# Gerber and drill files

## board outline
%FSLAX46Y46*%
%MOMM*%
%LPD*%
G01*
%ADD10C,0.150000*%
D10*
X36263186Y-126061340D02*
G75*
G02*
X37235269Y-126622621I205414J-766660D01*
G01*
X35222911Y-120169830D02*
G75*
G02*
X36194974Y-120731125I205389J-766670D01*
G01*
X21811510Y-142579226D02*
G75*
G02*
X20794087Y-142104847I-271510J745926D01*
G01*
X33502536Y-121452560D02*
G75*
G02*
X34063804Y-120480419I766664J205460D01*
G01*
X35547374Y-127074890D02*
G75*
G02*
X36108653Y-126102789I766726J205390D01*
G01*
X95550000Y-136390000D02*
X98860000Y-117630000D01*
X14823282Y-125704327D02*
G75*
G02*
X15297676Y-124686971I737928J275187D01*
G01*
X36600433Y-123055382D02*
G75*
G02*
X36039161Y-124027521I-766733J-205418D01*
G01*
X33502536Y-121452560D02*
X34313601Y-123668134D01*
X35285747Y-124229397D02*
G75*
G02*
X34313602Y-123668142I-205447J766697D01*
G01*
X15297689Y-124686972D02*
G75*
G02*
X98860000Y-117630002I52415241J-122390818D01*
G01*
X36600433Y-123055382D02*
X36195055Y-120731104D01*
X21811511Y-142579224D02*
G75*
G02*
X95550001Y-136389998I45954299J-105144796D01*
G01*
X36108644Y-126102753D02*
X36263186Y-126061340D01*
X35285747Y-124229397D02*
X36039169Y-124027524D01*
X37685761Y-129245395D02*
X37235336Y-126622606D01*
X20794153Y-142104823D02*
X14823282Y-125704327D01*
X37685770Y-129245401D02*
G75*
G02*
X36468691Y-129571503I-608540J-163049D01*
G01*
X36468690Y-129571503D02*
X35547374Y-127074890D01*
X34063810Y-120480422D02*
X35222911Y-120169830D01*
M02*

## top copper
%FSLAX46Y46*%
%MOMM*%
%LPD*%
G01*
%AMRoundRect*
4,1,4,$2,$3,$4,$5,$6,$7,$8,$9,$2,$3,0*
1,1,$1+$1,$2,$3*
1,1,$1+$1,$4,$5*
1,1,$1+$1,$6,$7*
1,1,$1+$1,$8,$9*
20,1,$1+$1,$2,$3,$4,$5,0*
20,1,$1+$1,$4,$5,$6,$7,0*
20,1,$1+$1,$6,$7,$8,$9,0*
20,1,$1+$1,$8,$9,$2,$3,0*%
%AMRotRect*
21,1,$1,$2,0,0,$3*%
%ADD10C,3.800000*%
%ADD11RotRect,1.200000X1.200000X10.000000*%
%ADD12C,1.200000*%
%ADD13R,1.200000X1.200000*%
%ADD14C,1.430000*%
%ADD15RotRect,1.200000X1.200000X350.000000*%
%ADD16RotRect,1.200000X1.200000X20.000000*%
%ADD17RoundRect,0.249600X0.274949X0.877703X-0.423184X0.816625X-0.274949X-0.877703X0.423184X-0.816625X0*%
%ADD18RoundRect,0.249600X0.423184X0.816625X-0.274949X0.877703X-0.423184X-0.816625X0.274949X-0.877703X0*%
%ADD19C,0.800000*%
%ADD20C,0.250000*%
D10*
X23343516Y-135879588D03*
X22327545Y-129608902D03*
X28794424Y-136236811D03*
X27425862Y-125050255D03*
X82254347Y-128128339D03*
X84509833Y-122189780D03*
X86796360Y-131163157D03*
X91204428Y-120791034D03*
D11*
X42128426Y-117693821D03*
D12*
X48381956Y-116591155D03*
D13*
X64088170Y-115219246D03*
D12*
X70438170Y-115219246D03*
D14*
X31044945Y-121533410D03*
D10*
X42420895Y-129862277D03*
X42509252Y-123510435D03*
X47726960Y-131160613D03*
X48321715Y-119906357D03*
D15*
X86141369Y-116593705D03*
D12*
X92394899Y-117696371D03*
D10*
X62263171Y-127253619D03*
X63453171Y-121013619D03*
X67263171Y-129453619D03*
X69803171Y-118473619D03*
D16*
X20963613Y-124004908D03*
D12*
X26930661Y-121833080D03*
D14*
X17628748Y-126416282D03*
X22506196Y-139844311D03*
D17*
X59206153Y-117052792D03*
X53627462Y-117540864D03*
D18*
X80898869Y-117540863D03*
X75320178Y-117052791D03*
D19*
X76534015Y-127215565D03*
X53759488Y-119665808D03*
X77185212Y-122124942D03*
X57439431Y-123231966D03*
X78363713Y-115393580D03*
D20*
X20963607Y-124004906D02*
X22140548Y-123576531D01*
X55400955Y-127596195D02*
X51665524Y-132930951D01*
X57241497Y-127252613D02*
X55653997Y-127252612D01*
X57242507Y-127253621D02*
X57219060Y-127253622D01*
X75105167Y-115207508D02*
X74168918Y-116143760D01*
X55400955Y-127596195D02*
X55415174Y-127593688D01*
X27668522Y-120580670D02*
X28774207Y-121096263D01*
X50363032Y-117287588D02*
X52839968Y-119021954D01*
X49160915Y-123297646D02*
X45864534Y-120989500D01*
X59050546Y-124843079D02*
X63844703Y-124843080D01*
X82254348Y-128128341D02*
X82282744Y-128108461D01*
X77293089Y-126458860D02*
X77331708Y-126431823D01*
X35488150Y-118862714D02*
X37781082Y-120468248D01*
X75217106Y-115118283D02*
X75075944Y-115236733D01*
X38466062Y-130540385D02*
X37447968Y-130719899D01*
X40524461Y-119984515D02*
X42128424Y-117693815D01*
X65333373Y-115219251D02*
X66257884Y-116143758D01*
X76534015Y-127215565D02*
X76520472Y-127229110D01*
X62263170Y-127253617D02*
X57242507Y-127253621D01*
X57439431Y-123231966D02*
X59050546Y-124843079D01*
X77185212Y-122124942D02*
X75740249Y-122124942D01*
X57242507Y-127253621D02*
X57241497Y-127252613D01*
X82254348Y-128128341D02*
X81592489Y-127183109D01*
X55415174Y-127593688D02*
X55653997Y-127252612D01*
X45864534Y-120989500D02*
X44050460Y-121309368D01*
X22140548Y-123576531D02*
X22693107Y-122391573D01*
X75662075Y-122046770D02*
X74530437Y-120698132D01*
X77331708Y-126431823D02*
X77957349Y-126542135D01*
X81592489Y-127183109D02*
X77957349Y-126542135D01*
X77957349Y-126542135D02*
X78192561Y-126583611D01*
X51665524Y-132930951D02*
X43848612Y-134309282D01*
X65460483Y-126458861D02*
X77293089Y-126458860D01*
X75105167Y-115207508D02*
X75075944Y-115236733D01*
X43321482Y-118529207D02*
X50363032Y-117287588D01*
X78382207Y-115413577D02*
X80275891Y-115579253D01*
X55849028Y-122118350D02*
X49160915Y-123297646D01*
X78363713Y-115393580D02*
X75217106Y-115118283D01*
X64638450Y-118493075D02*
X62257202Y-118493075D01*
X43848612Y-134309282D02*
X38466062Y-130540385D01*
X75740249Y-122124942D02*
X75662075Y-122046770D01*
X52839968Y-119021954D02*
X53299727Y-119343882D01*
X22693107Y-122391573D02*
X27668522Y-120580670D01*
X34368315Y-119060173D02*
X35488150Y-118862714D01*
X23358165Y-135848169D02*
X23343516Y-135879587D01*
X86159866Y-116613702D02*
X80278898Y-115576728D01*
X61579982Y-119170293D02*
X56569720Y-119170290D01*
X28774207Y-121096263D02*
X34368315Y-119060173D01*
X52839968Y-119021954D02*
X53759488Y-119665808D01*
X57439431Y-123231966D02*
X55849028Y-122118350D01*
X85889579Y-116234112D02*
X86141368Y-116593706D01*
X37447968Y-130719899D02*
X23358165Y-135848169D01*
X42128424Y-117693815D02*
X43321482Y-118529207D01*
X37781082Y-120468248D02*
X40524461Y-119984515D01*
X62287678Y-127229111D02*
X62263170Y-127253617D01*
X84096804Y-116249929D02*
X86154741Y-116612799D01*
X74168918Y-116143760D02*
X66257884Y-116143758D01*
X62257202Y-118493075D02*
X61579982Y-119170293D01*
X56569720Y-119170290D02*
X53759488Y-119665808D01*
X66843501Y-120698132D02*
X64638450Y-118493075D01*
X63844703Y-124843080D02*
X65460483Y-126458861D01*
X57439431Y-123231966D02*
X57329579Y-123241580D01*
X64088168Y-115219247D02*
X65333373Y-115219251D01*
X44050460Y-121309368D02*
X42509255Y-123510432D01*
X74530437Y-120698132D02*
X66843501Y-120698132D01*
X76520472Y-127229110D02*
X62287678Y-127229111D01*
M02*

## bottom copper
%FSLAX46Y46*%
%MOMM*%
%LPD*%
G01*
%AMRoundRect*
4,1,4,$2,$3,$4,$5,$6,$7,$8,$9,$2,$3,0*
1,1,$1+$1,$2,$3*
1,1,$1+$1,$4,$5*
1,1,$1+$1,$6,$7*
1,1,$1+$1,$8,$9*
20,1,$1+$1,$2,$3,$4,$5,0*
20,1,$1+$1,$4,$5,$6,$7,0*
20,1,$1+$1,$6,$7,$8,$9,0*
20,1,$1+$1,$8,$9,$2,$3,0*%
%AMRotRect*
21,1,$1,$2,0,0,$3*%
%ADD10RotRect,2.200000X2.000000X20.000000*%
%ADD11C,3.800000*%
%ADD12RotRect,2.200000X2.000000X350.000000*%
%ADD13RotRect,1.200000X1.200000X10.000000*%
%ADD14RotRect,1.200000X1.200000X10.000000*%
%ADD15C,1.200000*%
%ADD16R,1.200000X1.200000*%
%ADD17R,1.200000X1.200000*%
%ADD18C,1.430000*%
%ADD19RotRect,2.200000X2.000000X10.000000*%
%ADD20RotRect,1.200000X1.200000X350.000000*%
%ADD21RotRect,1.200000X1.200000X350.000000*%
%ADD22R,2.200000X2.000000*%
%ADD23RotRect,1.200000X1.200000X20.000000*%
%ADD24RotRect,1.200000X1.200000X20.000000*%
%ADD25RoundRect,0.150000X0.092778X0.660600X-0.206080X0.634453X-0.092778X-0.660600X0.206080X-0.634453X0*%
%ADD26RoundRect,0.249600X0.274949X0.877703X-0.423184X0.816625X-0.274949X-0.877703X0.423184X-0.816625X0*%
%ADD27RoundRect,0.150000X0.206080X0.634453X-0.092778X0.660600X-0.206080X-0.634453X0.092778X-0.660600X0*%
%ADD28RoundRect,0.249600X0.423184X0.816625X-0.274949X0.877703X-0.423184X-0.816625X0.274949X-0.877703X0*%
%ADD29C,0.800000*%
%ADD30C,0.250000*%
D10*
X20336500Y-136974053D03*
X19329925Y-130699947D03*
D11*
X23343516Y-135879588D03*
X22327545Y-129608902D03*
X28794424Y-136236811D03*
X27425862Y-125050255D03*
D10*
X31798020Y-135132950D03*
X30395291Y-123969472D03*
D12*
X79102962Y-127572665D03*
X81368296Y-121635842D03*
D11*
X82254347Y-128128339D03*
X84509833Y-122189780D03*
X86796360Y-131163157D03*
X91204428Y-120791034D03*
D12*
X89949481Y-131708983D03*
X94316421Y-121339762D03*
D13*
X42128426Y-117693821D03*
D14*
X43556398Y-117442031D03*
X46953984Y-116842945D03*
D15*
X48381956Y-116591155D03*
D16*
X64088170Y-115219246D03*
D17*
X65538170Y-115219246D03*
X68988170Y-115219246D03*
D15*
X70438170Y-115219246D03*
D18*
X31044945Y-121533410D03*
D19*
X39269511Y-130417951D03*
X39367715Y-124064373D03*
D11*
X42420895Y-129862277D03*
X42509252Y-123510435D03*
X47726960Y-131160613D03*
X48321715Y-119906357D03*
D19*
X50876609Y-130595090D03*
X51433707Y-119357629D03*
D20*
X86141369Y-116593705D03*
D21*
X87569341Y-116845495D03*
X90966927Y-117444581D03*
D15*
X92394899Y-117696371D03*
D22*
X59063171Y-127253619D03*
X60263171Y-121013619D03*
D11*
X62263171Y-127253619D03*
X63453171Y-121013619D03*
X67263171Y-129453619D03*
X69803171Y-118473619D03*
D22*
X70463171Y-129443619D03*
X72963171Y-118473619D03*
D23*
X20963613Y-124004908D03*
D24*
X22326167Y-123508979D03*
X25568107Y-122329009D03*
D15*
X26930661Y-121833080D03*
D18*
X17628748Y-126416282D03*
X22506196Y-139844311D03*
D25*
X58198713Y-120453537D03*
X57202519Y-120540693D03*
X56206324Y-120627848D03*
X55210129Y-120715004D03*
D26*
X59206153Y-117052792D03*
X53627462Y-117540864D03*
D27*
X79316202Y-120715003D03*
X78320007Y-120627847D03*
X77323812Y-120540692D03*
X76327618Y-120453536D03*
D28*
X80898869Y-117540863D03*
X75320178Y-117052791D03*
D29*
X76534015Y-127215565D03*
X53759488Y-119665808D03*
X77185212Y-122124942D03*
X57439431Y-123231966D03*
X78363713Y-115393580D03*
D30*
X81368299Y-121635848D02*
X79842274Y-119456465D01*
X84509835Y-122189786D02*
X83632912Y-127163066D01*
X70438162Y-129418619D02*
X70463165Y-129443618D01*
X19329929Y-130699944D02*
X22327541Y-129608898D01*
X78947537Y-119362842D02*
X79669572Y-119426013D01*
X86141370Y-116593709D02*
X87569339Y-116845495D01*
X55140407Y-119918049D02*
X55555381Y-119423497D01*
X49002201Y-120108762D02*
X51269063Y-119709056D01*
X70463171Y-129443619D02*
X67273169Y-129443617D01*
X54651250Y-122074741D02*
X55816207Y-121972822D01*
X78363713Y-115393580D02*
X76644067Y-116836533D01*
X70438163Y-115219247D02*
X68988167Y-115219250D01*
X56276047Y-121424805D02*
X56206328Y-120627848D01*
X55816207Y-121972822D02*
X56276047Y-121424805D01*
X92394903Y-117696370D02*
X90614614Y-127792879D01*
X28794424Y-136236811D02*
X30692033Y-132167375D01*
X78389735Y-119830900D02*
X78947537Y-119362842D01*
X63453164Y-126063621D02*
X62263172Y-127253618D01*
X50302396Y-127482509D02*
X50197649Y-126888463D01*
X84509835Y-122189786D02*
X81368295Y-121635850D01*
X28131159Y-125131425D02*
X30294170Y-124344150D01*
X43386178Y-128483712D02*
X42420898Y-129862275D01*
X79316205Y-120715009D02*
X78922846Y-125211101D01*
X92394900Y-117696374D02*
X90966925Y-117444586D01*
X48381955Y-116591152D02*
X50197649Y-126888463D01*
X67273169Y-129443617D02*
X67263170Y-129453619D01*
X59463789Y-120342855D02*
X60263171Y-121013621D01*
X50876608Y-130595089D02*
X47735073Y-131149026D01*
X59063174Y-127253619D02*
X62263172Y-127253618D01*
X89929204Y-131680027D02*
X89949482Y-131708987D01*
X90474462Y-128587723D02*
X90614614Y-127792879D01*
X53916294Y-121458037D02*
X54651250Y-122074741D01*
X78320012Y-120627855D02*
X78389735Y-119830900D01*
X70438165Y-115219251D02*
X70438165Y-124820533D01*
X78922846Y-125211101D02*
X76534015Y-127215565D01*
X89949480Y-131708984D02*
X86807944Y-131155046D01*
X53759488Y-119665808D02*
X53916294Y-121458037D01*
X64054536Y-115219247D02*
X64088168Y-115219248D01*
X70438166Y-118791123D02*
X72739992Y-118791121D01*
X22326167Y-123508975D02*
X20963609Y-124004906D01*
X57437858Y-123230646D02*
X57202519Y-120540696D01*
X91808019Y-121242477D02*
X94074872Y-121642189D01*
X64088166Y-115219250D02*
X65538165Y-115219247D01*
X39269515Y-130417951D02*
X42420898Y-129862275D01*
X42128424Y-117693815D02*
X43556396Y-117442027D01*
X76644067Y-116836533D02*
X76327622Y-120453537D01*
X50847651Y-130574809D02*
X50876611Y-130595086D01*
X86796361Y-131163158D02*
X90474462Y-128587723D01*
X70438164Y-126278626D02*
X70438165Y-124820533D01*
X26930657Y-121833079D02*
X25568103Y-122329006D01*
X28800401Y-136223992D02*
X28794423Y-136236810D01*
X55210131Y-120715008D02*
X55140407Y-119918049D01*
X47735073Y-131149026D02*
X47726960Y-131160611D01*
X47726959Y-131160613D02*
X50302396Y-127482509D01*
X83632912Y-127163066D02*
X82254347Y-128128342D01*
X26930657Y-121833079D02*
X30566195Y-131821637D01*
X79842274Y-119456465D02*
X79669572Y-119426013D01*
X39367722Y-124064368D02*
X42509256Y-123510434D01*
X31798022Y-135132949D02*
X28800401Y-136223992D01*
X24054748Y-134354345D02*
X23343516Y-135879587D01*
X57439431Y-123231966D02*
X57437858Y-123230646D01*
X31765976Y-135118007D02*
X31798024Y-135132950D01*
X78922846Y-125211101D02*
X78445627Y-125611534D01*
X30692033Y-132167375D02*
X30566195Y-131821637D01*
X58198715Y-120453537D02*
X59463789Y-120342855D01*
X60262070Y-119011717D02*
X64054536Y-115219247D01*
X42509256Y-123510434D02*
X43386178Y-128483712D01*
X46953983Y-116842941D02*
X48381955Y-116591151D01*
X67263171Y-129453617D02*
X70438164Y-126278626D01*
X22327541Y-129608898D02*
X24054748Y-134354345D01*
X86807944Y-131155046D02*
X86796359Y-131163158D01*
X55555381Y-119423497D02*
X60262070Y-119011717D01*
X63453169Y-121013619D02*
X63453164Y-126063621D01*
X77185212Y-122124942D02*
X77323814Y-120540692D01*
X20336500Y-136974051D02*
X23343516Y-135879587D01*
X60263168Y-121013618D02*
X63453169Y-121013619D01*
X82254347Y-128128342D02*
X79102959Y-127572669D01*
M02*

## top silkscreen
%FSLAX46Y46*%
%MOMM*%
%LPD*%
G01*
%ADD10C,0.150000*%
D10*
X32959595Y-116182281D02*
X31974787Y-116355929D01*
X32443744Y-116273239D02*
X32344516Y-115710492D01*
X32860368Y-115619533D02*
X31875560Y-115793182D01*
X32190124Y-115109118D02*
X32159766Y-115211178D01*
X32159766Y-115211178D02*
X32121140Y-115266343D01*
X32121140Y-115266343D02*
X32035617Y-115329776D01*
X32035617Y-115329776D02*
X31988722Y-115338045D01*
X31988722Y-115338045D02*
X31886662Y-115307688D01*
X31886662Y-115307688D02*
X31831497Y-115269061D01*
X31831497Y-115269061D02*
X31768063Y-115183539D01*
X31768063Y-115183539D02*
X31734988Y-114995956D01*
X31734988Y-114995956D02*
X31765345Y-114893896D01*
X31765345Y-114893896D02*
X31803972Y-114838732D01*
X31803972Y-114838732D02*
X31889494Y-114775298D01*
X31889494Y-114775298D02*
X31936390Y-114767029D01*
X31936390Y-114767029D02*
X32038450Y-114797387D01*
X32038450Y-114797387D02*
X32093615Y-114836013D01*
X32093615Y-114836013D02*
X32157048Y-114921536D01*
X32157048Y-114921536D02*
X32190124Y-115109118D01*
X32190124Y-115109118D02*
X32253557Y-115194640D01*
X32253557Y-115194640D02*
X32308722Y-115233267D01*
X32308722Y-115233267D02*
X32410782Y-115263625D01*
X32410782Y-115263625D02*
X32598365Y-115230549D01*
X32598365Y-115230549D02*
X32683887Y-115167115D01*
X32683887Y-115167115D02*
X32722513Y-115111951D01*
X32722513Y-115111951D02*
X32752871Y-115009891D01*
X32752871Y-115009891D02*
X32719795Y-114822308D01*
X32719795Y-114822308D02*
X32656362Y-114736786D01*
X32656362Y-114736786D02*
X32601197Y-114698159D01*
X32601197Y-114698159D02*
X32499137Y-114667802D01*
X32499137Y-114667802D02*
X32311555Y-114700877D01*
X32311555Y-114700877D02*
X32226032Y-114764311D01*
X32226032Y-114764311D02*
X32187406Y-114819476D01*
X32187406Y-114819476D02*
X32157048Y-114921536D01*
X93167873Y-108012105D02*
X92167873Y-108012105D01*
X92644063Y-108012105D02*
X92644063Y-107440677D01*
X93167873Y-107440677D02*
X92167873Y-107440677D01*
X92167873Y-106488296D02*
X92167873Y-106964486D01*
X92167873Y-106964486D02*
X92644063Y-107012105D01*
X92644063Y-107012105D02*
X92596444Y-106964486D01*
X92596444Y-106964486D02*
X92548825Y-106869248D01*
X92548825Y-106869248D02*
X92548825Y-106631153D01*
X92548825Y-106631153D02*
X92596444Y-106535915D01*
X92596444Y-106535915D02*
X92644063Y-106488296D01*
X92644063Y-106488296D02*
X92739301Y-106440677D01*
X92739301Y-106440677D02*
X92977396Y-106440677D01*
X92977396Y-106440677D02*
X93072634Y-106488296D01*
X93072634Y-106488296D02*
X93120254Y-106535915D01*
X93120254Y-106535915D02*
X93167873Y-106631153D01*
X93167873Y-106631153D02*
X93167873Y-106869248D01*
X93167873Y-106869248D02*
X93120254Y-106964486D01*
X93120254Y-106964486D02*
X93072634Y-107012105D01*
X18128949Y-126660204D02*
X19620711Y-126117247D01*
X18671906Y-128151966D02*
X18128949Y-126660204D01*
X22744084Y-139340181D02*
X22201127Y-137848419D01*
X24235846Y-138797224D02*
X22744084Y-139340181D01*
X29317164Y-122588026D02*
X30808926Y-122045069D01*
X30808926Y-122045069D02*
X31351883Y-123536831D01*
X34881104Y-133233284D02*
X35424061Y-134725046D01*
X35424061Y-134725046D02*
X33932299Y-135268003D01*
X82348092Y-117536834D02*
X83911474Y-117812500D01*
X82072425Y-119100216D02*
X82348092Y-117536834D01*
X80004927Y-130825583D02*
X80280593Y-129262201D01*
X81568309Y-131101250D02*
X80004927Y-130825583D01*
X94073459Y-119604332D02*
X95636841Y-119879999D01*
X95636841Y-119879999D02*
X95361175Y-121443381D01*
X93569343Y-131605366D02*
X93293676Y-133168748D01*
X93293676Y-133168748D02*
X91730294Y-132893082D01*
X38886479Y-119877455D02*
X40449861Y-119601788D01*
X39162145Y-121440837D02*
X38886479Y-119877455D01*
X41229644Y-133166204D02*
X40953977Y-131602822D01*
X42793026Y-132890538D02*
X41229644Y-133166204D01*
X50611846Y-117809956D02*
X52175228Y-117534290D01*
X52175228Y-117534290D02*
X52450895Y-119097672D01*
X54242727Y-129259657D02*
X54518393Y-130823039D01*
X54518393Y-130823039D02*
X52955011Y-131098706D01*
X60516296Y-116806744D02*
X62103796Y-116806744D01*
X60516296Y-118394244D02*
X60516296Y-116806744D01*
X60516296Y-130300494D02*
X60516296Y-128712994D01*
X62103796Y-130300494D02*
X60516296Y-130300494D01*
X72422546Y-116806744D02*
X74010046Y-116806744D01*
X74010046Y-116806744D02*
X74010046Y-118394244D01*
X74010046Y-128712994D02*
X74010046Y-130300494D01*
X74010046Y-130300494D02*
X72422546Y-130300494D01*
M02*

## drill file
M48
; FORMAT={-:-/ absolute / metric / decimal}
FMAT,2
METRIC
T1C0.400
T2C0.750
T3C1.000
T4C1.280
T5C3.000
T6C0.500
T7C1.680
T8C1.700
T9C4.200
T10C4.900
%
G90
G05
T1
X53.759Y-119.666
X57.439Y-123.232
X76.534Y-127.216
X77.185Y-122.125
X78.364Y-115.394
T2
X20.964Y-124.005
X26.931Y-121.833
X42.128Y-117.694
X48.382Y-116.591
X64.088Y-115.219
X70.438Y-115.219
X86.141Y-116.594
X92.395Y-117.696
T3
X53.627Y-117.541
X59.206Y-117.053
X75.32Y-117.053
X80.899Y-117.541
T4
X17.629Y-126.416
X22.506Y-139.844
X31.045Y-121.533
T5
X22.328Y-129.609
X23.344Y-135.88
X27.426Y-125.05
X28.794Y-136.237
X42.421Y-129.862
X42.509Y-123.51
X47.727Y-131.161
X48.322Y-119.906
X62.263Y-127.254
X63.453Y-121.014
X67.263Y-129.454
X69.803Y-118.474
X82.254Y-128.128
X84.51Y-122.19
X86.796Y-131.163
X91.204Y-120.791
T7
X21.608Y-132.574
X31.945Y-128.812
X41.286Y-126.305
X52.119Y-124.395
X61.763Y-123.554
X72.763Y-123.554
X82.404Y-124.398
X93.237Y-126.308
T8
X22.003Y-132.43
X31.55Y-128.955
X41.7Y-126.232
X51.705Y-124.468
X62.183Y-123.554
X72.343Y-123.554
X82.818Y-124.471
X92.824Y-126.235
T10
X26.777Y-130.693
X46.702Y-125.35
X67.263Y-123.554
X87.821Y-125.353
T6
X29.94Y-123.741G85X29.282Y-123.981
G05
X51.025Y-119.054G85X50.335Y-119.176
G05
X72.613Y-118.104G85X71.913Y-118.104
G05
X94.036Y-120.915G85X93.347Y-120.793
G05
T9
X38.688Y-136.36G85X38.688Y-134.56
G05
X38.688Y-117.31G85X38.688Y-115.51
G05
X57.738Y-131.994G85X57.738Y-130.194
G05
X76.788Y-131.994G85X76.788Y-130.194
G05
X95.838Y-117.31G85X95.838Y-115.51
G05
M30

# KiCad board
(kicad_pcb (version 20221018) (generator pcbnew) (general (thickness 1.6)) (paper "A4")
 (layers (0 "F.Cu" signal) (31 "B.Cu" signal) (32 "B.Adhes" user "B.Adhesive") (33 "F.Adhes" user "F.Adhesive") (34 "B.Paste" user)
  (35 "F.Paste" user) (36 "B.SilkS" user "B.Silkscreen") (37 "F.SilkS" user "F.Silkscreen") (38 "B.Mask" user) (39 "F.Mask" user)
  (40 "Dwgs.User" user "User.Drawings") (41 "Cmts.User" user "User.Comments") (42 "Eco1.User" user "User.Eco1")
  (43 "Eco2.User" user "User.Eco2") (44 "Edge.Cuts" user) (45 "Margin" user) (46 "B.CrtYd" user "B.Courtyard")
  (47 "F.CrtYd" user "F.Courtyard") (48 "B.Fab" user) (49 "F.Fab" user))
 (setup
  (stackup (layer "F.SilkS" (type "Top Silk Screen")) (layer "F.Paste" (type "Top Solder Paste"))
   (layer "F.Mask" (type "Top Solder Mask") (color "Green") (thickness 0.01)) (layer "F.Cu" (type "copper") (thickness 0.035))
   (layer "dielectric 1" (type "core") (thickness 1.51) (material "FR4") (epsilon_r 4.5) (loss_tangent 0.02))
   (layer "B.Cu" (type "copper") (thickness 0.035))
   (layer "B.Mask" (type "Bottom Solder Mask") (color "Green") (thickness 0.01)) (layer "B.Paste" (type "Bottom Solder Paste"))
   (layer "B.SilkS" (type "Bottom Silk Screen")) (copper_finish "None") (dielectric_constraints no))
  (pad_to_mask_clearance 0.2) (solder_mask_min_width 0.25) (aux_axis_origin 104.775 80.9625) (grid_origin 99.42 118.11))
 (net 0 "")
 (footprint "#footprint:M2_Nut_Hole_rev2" (layer "F.Cu") (at 38.688167 135.459876 90)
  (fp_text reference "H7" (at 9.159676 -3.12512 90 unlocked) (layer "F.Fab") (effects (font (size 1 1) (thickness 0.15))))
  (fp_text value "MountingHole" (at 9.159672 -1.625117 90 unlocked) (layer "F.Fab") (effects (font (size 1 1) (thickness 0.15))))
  (pad "" np_thru_hole oval (at 0 0 90) (size 6 4.2) (drill oval 6 4.2) (layers "F&B.Cu" "*.Mask")))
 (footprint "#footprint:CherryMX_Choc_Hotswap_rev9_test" (layer "F.Cu") (at 26.776505 130.692625 20)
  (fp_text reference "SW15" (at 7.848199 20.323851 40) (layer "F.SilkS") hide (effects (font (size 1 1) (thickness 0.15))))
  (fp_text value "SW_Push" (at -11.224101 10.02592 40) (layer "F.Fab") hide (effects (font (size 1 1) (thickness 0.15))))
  (fp_line (start -6.746875 -6.746875) (end -5.159375 -6.746875) (stroke (width 0.15) (type solid)) (layer "F.SilkS"))
  (fp_line (start -6.746875 -5.159375) (end -6.746875 -6.746875) (stroke (width 0.15) (type solid)) (layer "F.SilkS"))
  (fp_line (start -6.746875 6.746875) (end -6.746875 5.159375) (stroke (width 0.15) (type solid)) (layer "F.SilkS"))
  (fp_line (start -5.159375 6.746875) (end -6.746875 6.746875) (stroke (width 0.15) (type solid)) (layer "F.SilkS"))
  (fp_line (start 5.159375 -6.746875) (end 6.746875 -6.746875) (stroke (width 0.15) (type solid)) (layer "F.SilkS"))
  (fp_line (start 6.746875 -6.746875) (end 6.746875 -5.159375) (stroke (width 0.15) (type solid)) (layer "F.SilkS"))
  (fp_line (start 6.746875 5.159375) (end 6.746875 6.746875) (stroke (width 0.15) (type solid)) (layer "F.SilkS"))
  (fp_line (start 6.746875 6.746875) (end 5.159375 6.746875) (stroke (width 0.15) (type solid)) (layer "F.SilkS"))
  (pad "" np_thru_hole circle (at -5.5 0 110) (size 1.68 1.68) (drill 1.68) (layers "F&B.Cu" "*.Mask"))
  (pad "" np_thru_hole circle (at -5.08 0 20) (size 1.7 1.7) (drill 1.7) (layers "*.Cu" "*.Mask"))
  (pad "" np_thru_hole circle (at 0 0 110) (size 4.9 4.9) (drill 4.9) (layers "F&B.Cu" "*.Mask"))
  (pad "" np_thru_hole oval (at 5 -5.45 200) (size 1.2 0.5) (drill oval 1.2 0.5) (layers "F&B.Cu" "*.Mask"))
  (pad "" np_thru_hole circle (at 5.08 0 20) (size 1.7 1.7) (drill 1.7) (layers "*.Cu" "*.Mask"))
  (pad "" np_thru_hole circle (at 5.5 0 110) (size 1.68 1.68) (drill 1.68) (layers "F&B.Cu" "*.Mask"))
  (pad "1" smd rect (at -8.2 3.7 20) (size 2.2 2) (layers "B.Cu" "B.Paste" "B.Mask"))
  (pad "1" smd rect (at -7 -2.54 20) (size 2.2 2) (layers "B.Cu" "B.Paste" "B.Mask"))
  (pad "1" thru_hole circle (at -5 3.7 110) (size 3.8 3.8) (drill 3) (layers "*.Cu" "B.Mask"))
  (pad "1" thru_hole circle (at -3.81 -2.54 200) (size 3.8 3.8) (drill 3) (layers "*.Cu" "B.Mask"))
  (pad "2" thru_hole circle (at 0 5.9 110) (size 3.8 3.8) (drill 3) (layers "*.Cu" "B.Mask"))
  (pad "2" thru_hole circle (at 2.54 -5.08 200) (size 3.8 3.8) (drill 3) (layers "*.Cu" "B.Mask"))
  (pad "2" smd rect (at 3.2 5.89 20) (size 2.2 2) (layers "B.Cu" "B.Paste" "B.Mask"))
  (pad "2" smd rect (at 5.7 -5.08 20) (size 2.2 2) (layers "B.Cu" "B.Paste" "B.Mask")))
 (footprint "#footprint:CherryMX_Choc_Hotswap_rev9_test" (layer "F.Cu") (at 87.820884 125.352791 -10)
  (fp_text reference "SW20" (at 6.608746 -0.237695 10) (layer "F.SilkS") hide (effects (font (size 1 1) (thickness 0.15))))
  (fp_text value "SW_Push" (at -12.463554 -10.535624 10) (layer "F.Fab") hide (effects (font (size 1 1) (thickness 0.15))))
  (fp_line (start -6.746875 -6.746875) (end -5.159375 -6.746875) (stroke (width 0.15) (type solid)) (layer "F.SilkS"))
  (fp_line (start -6.746875 -5.159375) (end -6.746875 -6.746875) (stroke (width 0.15) (type solid)) (layer "F.SilkS"))
  (fp_line (start -6.746875 6.746875) (end -6.746875 5.159375) (stroke (width 0.15) (type solid)) (layer "F.SilkS"))
  (fp_line (start -5.159375 6.746875) (end -6.746875 6.746875) (stroke (width 0.15) (type solid)) (layer "F.SilkS"))
  (fp_line (start 5.159375 -6.746875) (end 6.746875 -6.746875) (stroke (width 0.15) (type solid)) (layer "F.SilkS"))
  (fp_line (start 6.746875 -6.746875) (end 6.746875 -5.159375) (stroke (width 0.15) (type solid)) (layer "F.SilkS"))
  (fp_line (start 6.746875 5.159375) (end 6.746875 6.746875) (stroke (width 0.15) (type solid)) (layer "F.SilkS"))
  (fp_line (start 6.746875 6.746875) (end 5.159375 6.746875) (stroke (width 0.15) (type solid)) (layer "F.SilkS"))
  (pad "" np_thru_hole circle (at -5.5 0 80) (size 1.68 1.68) (drill 1.68) (layers "F&B.Cu" "*.Mask"))
  (pad "" np_thru_hole circle (at -5.08 0 350) (size 1.7 1.7) (drill 1.7) (layers "*.Cu" "*.Mask"))
  (pad "" np_thru_hole circle (at 0 0 80) (size 4.9 4.9) (drill 4.9) (layers "F&B.Cu" "*.Mask"))
  (pad "" np_thru_hole oval (at 5 -5.45 170) (size 1.2 0.5) (drill oval 1.2 0.5) (layers "F&B.Cu" "*.Mask"))
  (pad "" np_thru_hole circle (at 5.08 0 350) (size 1.7 1.7) (drill 1.7) (layers "*.Cu" "*.Mask"))
  (pad "" np_thru_hole circle (at 5.5 0 80) (size 1.68 1.68) (drill 1.68) (layers "F&B.Cu" "*.Mask"))
  (pad "1" smd rect (at -8.2 3.7 350) (size 2.2 2) (layers "B.Cu" "B.Paste" "B.Mask"))
  (pad "1" smd rect (at -7 -2.54 350) (size 2.2 2) (layers "B.Cu" "B.Paste" "B.Mask"))
  (pad "1" thru_hole circle (at -5 3.7 80) (size 3.8 3.8) (drill 3) (layers "*.Cu" "B.Mask"))
  (pad "1" thru_hole circle (at -3.81 -2.54 170) (size 3.8 3.8) (drill 3) (layers "*.Cu" "B.Mask"))
  (pad "2" thru_hole circle (at 0 5.9 80) (size 3.8 3.8) (drill 3) (layers "*.Cu" "B.Mask"))
  (pad "2" thru_hole circle (at 2.54 -5.08 170) (size 3.8 3.8) (drill 3) (layers "*.Cu" "B.Mask"))
  (pad "2" smd rect (at 3.2 5.89 350) (size 2.2 2) (layers "B.Cu" "B.Paste" "B.Mask"))
  (pad "2" smd rect (at 5.7 -5.08 350) (size 2.2 2) (layers "B.Cu" "B.Paste" "B.Mask")))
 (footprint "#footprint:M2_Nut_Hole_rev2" (layer "F.Cu") (at 76.788168 131.09425 90)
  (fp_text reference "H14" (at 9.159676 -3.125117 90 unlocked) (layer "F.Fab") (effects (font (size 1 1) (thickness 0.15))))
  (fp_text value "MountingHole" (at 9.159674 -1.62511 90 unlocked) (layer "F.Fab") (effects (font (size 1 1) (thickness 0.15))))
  (pad "" np_thru_hole oval (at 0 0 90) (size 6 4.2) (drill oval 6 4.2) (layers "F&B.Cu" "*.Mask")))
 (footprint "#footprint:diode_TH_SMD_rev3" (layer "F.Cu") (at 45.255191 117.142488 10)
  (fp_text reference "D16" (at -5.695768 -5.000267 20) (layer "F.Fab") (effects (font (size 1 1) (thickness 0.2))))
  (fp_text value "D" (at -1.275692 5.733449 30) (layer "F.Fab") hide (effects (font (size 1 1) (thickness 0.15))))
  (pad "1" thru_hole rect (at -3.175 0 10) (size 1.2 1.2) (drill 0.75) (layers "*.Cu" "B.Mask"))
  (pad "1" smd rect (at -1.725 0 10) (size 1.2 1.2) (layers "B.Cu" "B.Paste" "B.Mask"))
  (pad "2" smd rect (at 1.725 0 10) (size 1.2 1.2) (layers "B.Cu" "B.Paste" "B.Mask"))
  (pad "2" thru_hole circle (at 3.175 0 10) (size 1.2 1.2) (drill 0.75) (layers "*.Cu" "B.Mask")))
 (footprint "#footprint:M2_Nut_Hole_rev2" (layer "F.Cu") (at 38.688172 116.409876 90)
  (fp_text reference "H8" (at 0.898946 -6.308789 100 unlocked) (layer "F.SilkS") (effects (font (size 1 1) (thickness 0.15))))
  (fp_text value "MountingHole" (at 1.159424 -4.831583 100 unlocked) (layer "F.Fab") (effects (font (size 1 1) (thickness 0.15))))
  (pad "" np_thru_hole oval (at 0 0 90) (size 6 4.2) (drill oval 6 4.2) (layers "F&B.Cu" "*.Mask")))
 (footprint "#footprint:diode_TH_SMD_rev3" (layer "F.Cu") (at 67.26317 115.219246)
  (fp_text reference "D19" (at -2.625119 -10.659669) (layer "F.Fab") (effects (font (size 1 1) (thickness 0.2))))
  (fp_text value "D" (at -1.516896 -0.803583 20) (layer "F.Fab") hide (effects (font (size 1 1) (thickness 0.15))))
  (pad "1" thru_hole rect (at -3.175 0) (size 1.2 1.2) (drill 0.75) (layers "*.Cu" "B.Mask"))
  (pad "1" smd rect (at -1.725 0) (size 1.2 1.2) (layers "B.Cu" "B.Paste" "B.Mask"))
  (pad "2" smd rect (at 1.725 0) (size 1.2 1.2) (layers "B.Cu" "B.Paste" "B.Mask"))
  (pad "2" thru_hole circle (at 3.175 0) (size 1.2 1.2) (drill 0.75) (layers "*.Cu" "B.Mask")))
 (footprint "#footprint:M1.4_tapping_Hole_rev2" (layer "F.Cu") (at 31.044945 121.53341)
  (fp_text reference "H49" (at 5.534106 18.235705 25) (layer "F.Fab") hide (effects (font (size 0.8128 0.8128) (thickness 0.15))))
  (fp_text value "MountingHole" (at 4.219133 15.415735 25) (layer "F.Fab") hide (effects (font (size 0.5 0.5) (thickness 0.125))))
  (pad "" thru_hole circle (at 0 0) (size 1.43 1.43) (drill 1.28) (layers "*.Cu" "*.Mask")))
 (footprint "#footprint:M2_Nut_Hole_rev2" (layer "F.Cu") (at 95.83817 116.409867 90)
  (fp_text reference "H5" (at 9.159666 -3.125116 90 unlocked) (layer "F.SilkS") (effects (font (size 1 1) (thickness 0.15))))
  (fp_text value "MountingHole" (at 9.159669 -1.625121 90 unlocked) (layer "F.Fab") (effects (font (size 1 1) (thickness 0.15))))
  (pad "" np_thru_hole oval (at 0 0 90) (size 6 4.2) (drill oval 6 4.2) (layers "F&B.Cu" "*.Mask")))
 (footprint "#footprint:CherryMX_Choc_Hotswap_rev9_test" (layer "F.Cu") (at 46.702436 125.350247 10)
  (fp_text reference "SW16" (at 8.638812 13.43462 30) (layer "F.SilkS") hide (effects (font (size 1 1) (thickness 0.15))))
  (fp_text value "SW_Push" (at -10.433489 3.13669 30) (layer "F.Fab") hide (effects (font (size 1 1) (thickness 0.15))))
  (fp_line (start -6.746875 -6.746875) (end -5.159375 -6.746875) (stroke (width 0.15) (type solid)) (layer "F.SilkS"))
  (fp_line (start -6.746875 -5.159375) (end -6.746875 -6.746875) (stroke (width 0.15) (type solid)) (layer "F.SilkS"))
  (fp_line (start -6.746875 6.746875) (end -6.746875 5.159375) (stroke (width 0.15) (type solid)) (layer "F.SilkS"))
  (fp_line (start -5.159375 6.746875) (end -6.746875 6.746875) (stroke (width 0.15) (type solid)) (layer "F.SilkS"))
  (fp_line (start 5.159375 -6.746875) (end 6.746875 -6.746875) (stroke (width 0.15) (type solid)) (layer "F.SilkS"))
  (fp_line (start 6.746875 -6.746875) (end 6.746875 -5.159375) (stroke (width 0.15) (type solid)) (layer "F.SilkS"))
  (fp_line (start 6.746875 5.159375) (end 6.746875 6.746875) (stroke (width 0.15) (type solid)) (layer "F.SilkS"))
  (fp_line (start 6.746875 6.746875) (end 5.159375 6.746875) (stroke (width 0.15) (type solid)) (layer "F.SilkS"))
  (pad "" np_thru_hole circle (at -5.5 0 100) (size 1.68 1.68) (drill 1.68) (layers "F&B.Cu" "*.Mask"))
  (pad "" np_thru_hole circle (at -5.08 0 10) (size 1.7 1.7) (drill 1.7) (layers "*.Cu" "*.Mask"))
  (pad "" np_thru_hole circle (at 0 0 100) (size 4.9 4.9) (drill 4.9) (layers "F&B.Cu" "*.Mask"))
  (pad "" np_thru_hole oval (at 5 -5.45 190) (size 1.2 0.5) (drill oval 1.2 0.5) (layers "F&B.Cu" "*.Mask"))
  (pad "" np_thru_hole circle (at 5.08 0 10) (size 1.7 1.7) (drill 1.7) (layers "*.Cu" "*.Mask"))
  (pad "" np_thru_hole circle (at 5.5 0 100) (size 1.68 1.68) (drill 1.68) (layers "F&B.Cu" "*.Mask"))
  (pad "1" smd rect (at -8.2 3.7 10) (size 2.2 2) (layers "B.Cu" "B.Paste" "B.Mask"))
  (pad "1" smd rect (at -7 -2.54 10) (size 2.2 2) (layers "B.Cu" "B.Paste" "B.Mask"))
  (pad "1" thru_hole circle (at -5 3.7 100) (size 3.8 3.8) (drill 3) (layers "*.Cu" "B.Mask"))
  (pad "1" thru_hole circle (at -3.81 -2.54 190) (size 3.8 3.8) (drill 3) (layers "*.Cu" "B.Mask"))
  (pad "2" thru_hole circle (at 0 5.9 100) (size 3.8 3.8) (drill 3) (layers "*.Cu" "B.Mask"))
  (pad "2" thru_hole circle (at 2.54 -5.08 190) (size 3.8 3.8) (drill 3) (layers "*.Cu" "B.Mask"))
  (pad "2" smd rect (at 3.2 5.89 10) (size 2.2 2) (layers "B.Cu" "B.Paste" "B.Mask"))
  (pad "2" smd rect (at 5.7 -5.08 10) (size 2.2 2) (layers "B.Cu" "B.Paste" "B.Mask")))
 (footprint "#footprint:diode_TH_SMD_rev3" (layer "F.Cu") (at 89.268134 117.145038 -10)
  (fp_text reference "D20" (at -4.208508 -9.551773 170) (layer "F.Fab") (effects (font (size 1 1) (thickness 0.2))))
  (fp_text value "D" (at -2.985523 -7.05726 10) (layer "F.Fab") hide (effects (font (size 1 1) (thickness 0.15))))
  (pad "1" thru_hole rect (at -3.175 0 350) (size 1.2 1.2) (drill 0.75) (layers "*.Cu" "B.Mask"))
  (pad "1" smd rect (at -1.725 0 350) (size 1.2 1.2) (layers "B.Cu" "B.Paste" "B.Mask"))
  (pad "2" smd rect (at 1.725 0 350) (size 1.2 1.2) (layers "B.Cu" "B.Paste" "B.Mask"))
  (pad "2" thru_hole circle (at 3.175 0 350) (size 1.2 1.2) (drill 0.75) (layers "*.Cu" "B.Mask")))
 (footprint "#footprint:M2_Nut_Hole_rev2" (layer "F.Cu") (at 57.738174 131.094247 90)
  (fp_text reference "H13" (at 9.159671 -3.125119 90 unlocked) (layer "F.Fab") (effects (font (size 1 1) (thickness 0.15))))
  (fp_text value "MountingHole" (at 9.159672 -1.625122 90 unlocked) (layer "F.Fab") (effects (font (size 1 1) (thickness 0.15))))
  (pad "" np_thru_hole oval (at 0 0 90) (size 6 4.2) (drill oval 6 4.2) (layers "F&B.Cu" "*.Mask")))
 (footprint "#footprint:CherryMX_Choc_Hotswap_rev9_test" (layer "F.Cu") (at 67.263171 123.553619)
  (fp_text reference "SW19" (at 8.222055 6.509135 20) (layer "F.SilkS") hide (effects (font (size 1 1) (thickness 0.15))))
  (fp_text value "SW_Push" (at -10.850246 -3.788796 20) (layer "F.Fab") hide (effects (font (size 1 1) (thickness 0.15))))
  (fp_line (start -6.746875 -6.746875) (end -5.159375 -6.746875) (stroke (width 0.15) (type solid)) (layer "F.SilkS"))
  (fp_line (start -6.746875 -5.159375) (end -6.746875 -6.746875) (stroke (width 0.15) (type solid)) (layer "F.SilkS"))
  (fp_line (start -6.746875 6.746875) (end -6.746875 5.159375) (stroke (width 0.15) (type solid)) (layer "F.SilkS"))
  (fp_line (start -5.159375 6.746875) (end -6.746875 6.746875) (stroke (width 0.15) (type solid)) (layer "F.SilkS"))
  (fp_line (start 5.159375 -6.746875) (end 6.746875 -6.746875) (stroke (width 0.15) (type solid)) (layer "F.SilkS"))
  (fp_line (start 6.746875 -6.746875) (end 6.746875 -5.159375) (stroke (width 0.15) (type solid)) (layer "F.SilkS"))
  (fp_line (start 6.746875 5.159375) (end 6.746875 6.746875) (stroke (width 0.15) (type solid)) (layer "F.SilkS"))
  (fp_line (start 6.746875 6.746875) (end 5.159375 6.746875) (stroke (width 0.15) (type solid)) (layer "F.SilkS"))
  (pad "" np_thru_hole circle (at -5.5 0 90) (size 1.68 1.68) (drill 1.68) (layers "F&B.Cu" "*.Mask"))
  (pad "" np_thru_hole circle (at -5.08 0) (size 1.7 1.7) (drill 1.7) (layers "*.Cu" "*.Mask"))
  (pad "" np_thru_hole circle (at 0 0 90) (size 4.9 4.9) (drill 4.9) (layers "F&B.Cu" "*.Mask"))
  (pad "" np_thru_hole oval (at 5 -5.45 180) (size 1.2 0.5) (drill oval 1.2 0.5) (layers "F&B.Cu" "*.Mask"))
  (pad "" np_thru_hole circle (at 5.08 0) (size 1.7 1.7) (drill 1.7) (layers "*.Cu" "*.Mask"))
  (pad "" np_thru_hole circle (at 5.5 0 90) (size 1.68 1.68) (drill 1.68) (layers "F&B.Cu" "*.Mask"))
  (pad "1" smd rect (at -8.2 3.7) (size 2.2 2) (layers "B.Cu" "B.Paste" "B.Mask"))
  (pad "1" smd rect (at -7 -2.54) (size 2.2 2) (layers "B.Cu" "B.Paste" "B.Mask"))
  (pad "1" thru_hole circle (at -5 3.7 90) (size 3.8 3.8) (drill 3) (layers "*.Cu" "B.Mask"))
  (pad "1" thru_hole circle (at -3.81 -2.54 180) (size 3.8 3.8) (drill 3) (layers "*.Cu" "B.Mask"))
  (pad "2" thru_hole circle (at 0 5.9 90) (size 3.8 3.8) (drill 3) (layers "*.Cu" "B.Mask"))
  (pad "2" thru_hole circle (at 2.54 -5.08 180) (size 3.8 3.8) (drill 3) (layers "*.Cu" "B.Mask"))
  (pad "2" smd rect (at 3.2 5.89) (size 2.2 2) (layers "B.Cu" "B.Paste" "B.Mask"))
  (pad "2" smd rect (at 5.7 -5.08) (size 2.2 2) (layers "B.Cu" "B.Paste" "B.Mask")))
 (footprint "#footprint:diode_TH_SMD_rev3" (layer "F.Cu") (at 23.947137 122.918994 20)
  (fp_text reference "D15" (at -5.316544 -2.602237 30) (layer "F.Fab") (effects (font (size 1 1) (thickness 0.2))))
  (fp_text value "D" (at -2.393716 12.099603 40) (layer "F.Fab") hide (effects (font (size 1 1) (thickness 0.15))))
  (pad "1" thru_hole rect (at -3.175 0 20) (size 1.2 1.2) (drill 0.75) (layers "*.Cu" "B.Mask"))
  (pad "1" smd rect (at -1.725 0 20) (size 1.2 1.2) (layers "B.Cu" "B.Paste" "B.Mask"))
  (pad "2" smd rect (at 1.725 0 20) (size 1.2 1.2) (layers "B.Cu" "B.Paste" "B.Mask"))
  (pad "2" thru_hole circle (at 3.175 0 20) (size 1.2 1.2) (drill 0.75) (layers "*.Cu" "B.Mask")))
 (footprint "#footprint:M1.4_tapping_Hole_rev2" (layer "F.Cu") (at 17.628748 126.416282)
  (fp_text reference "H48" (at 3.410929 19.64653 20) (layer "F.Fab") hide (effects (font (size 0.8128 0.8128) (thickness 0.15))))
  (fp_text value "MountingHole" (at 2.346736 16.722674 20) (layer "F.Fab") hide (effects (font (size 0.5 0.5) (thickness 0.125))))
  (pad "" thru_hole circle (at 0 0) (size 1.43 1.43) (drill 1.28) (layers "*.Cu" "*.Mask")))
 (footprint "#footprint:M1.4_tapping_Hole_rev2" (layer "F.Cu") (at 22.506196 139.844311)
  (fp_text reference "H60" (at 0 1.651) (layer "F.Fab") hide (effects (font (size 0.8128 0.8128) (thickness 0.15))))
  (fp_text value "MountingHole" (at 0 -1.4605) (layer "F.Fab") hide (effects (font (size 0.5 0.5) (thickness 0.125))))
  (pad "" thru_hole circle (at 0 0) (size 1.43 1.43) (drill 1.28) (layers "*.Cu" "*.Mask")))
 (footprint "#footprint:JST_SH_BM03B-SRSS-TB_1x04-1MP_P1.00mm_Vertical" (layer "B.Cu") (at 56.547541 118.79112 -175)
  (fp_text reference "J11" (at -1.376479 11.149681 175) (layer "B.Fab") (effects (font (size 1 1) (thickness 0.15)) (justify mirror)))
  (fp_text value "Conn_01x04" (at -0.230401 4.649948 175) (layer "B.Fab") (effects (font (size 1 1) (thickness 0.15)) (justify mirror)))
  (pad "1" smd roundrect (at -1.5 -1.8 185) (size 0.6 1.6) (layers "B.Cu" "B.Paste" "B.Mask") (roundrect_rratio 0.25))
  (pad "2" smd roundrect (at -0.5 -1.8 185) (size 0.6 1.6) (layers "B.Cu" "B.Paste" "B.Mask") (roundrect_rratio 0.25))
  (pad "3" smd roundrect (at 0.5 -1.8 185) (size 0.6 1.6) (layers "B.Cu" "B.Paste" "B.Mask") (roundrect_rratio 0.25))
  (pad "4" smd roundrect (at 1.5 -1.8 185) (size 0.6 1.6) (layers "B.Cu" "B.Paste" "B.Mask") (roundrect_rratio 0.25))
  (pad "MP" thru_hole roundrect (at -2.8 1.5 185) (size 1.2 2.2) (drill 1) (layers "*.Cu" "*.Mask") (roundrect_rratio 0.208))
  (pad "MP" thru_hole roundrect (at 2.8 1.5 185) (size 1.2 2.2) (drill 1) (layers "*.Cu" "*.Mask") (roundrect_rratio 0.208)))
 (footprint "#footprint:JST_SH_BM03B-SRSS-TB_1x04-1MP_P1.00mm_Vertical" (layer "B.Cu") (at 77.97879 118.791119 175)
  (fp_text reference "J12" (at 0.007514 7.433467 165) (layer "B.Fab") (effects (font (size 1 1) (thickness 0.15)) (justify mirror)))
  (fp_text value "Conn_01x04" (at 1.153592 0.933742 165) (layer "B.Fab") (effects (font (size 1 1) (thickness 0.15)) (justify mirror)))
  (pad "1" smd roundrect (at -1.5 -1.8 175) (size 0.6 1.6) (layers "B.Cu" "B.Paste" "B.Mask") (roundrect_rratio 0.25))
  (pad "2" smd roundrect (at -0.5 -1.8 175) (size 0.6 1.6) (layers "B.Cu" "B.Paste" "B.Mask") (roundrect_rratio 0.25))
  (pad "3" smd roundrect (at 0.5 -1.8 175) (size 0.6 1.6) (layers "B.Cu" "B.Paste" "B.Mask") (roundrect_rratio 0.25))
  (pad "4" smd roundrect (at 1.5 -1.8 175) (size 0.6 1.6) (layers "B.Cu" "B.Paste" "B.Mask") (roundrect_rratio 0.25))
  (pad "MP" thru_hole roundrect (at -2.8 1.5 175) (size 1.2 2.2) (drill 1) (layers "*.Cu" "*.Mask") (roundrect_rratio 0.208))
  (pad "MP" thru_hole roundrect (at 2.8 1.5 175) (size 1.2 2.2) (drill 1) (layers "*.Cu" "*.Mask") (roundrect_rratio 0.208)))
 (gr_arc (start 36.263186 126.06134) (mid 36.865502 126.140633) (end 37.235335 126.622603) (stroke (width 0.15) (type solid))
  (layer "Edge.Cuts"))
 (gr_arc (start 35.222911 120.16983) (mid 35.825227 120.249129) (end 36.195056 120.731103) (stroke (width 0.15) (type solid))
  (layer "Edge.Cuts"))
 (gr_arc (start 21.81151 142.579226) (mid 21.204579 142.552726) (end 20.794153 142.104823) (stroke (width 0.15) (type solid))
  (layer "Edge.Cuts"))
 (gr_arc (start 33.502536 121.45256) (mid 33.581834 120.850249) (end 34.063805 120.480423) (stroke (width 0.15) (type solid))
  (layer "Edge.Cuts"))
 (gr_arc (start 35.547374 127.07489) (mid 35.626672 126.472578) (end 36.108643 126.102751) (stroke (width 0.15) (type solid))
  (layer "Edge.Cuts"))
 (gr_line (start 95.55 136.39) (end 98.86 117.63) (stroke (width 0.15) (type solid)) (layer "Edge.Cuts"))
 (gr_arc (start 14.823282 125.704327) (mid 14.847425 125.0963) (end 15.297674 124.686966) (stroke (width 0.15) (type solid))
  (layer "Edge.Cuts"))
 (gr_arc (start 36.600433 123.055382) (mid 36.521135 123.657697) (end 36.039162 124.027525) (stroke (width 0.15) (type solid))
  (layer "Edge.Cuts"))
 (gr_line (start 33.502536 121.45256) (end 34.313601 123.668134) (stroke (width 0.15) (type solid)) (layer "Edge.Cuts"))
 (gr_arc (start 35.285747 124.229397) (mid 34.683437 124.150105) (end 34.313608 123.66814) (stroke (width 0.15) (type solid))
  (layer "Edge.Cuts"))
 (gr_arc (start 15.297689 124.686972) (mid 56.508735 114.407763) (end 98.86 117.63) (stroke (width 0.15) (type solid)) (layer "Edge.Cuts"))
 (gr_line (start 36.600433 123.055382) (end 36.195055 120.731104) (stroke (width 0.15) (type solid)) (layer "Edge.Cuts"))
 (gr_arc (start 21.811511 142.579224) (mid 58.168162 133.37757) (end 95.55 136.39) (stroke (width 0.15) (type solid)) (layer "Edge.Cuts"))
 (gr_line (start 36.108644 126.102753) (end 36.263186 126.06134) (stroke (width 0.15) (type solid)) (layer "Edge.Cuts"))
 (gr_line (start 35.285747 124.229397) (end 36.039169 124.027524) (stroke (width 0.15) (type solid)) (layer "Edge.Cuts"))
 (gr_line (start 37.685761 129.245395) (end 37.235336 126.622606) (stroke (width 0.15) (type solid)) (layer "Edge.Cuts"))
 (gr_line (start 20.794153 142.104823) (end 14.823282 125.704327) (stroke (width 0.15) (type solid)) (layer "Edge.Cuts"))
 (gr_arc (start 37.68577 129.245401) (mid 37.240281 130.016992) (end 36.46869 129.571503) (stroke (width 0.15) (type solid))
  (layer "Edge.Cuts"))
 (gr_line (start 36.46869 129.571503) (end 35.547374 127.07489) (stroke (width 0.15) (type solid)) (layer "Edge.Cuts"))
 (gr_line (start 34.06381 120.480422) (end 35.222911 120.16983) (stroke (width 0.15) (type solid)) (layer "Edge.Cuts"))
 (segment (start 20.963607 124.004906) (end 22.140548 123.576531) (width 0.25) (layer "F.Cu") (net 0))
 (segment (start 55.400955 127.596195) (end 51.665524 132.930951) (width 0.25) (layer "F.Cu") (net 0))
 (segment (start 57.241497 127.252613) (end 55.653997 127.252612) (width 0.25) (layer "F.Cu") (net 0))
 (segment (start 57.242507 127.253621) (end 57.21906 127.253622) (width 0.25) (layer "F.Cu") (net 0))
 (segment (start 75.105167 115.207508) (end 74.168918 116.14376) (width 0.25) (layer "F.Cu") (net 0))
 (segment (start 55.400955 127.596195) (end 55.415174 127.593688) (width 0.25) (layer "F.Cu") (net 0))
 (segment (start 27.668522 120.58067) (end 28.774207 121.096263) (width 0.25) (layer "F.Cu") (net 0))
 (segment (start 50.363032 117.287588) (end 52.839968 119.021954) (width 0.25) (layer "F.Cu") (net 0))
 (segment (start 49.160915 123.297646) (end 45.864534 120.9895) (width 0.25) (layer "F.Cu") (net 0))
 (segment (start 59.050546 124.843079) (end 63.844703 124.84308) (width 0.25) (layer "F.Cu") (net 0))
 (segment (start 82.254348 128.128341) (end 82.282744 128.108461) (width 0.25) (layer "F.Cu") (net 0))
 (segment (start 77.293089 126.45886) (end 77.331708 126.431823) (width 0.25) (layer "F.Cu") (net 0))
 (segment (start 35.48815 118.862714) (end 37.781082 120.468248) (width 0.25) (layer "F.Cu") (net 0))
 (segment (start 75.217106 115.118283) (end 75.075944 115.236733) (width 0.25) (layer "F.Cu") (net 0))
 (segment (start 38.466062 130.540385) (end 37.447968 130.719899) (width 0.25) (layer "F.Cu") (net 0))
 (segment (start 40.524461 119.984515) (end 42.128424 117.693815) (width 0.25) (layer "F.Cu") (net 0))
 (segment (start 65.333373 115.219251) (end 66.257884 116.143758) (width 0.25) (layer "F.Cu") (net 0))
 (segment (start 76.534015 127.215565) (end 76.520472 127.22911) (width 0.25) (layer "F.Cu") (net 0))
 (segment (start 62.26317 127.253617) (end 57.242507 127.253621) (width 0.25) (layer "F.Cu") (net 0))
 (segment (start 57.439431 123.231966) (end 59.050546 124.843079) (width 0.25) (layer "F.Cu") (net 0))
 (segment (start 77.185212 122.124942) (end 75.740249 122.124942) (width 0.25) (layer "F.Cu") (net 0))
 (segment (start 57.242507 127.253621) (end 57.241497 127.252613) (width 0.25) (layer "F.Cu") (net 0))
 (segment (start 82.254348 128.128341) (end 81.592489 127.183109) (width 0.25) (layer "F.Cu") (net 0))
 (segment (start 55.415174 127.593688) (end 55.653997 127.252612) (width 0.25) (layer "F.Cu") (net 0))
 (segment (start 45.864534 120.9895) (end 44.05046 121.309368) (width 0.25) (layer "F.Cu") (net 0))
 (segment (start 22.140548 123.576531) (end 22.693107 122.391573) (width 0.25) (layer "F.Cu") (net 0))
 (segment (start 75.662075 122.04677) (end 74.530437 120.698132) (width 0.25) (layer "F.Cu") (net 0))
 (segment (start 77.331708 126.431823) (end 77.957349 126.542135) (width 0.25) (layer "F.Cu") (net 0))
 (segment (start 81.592489 127.183109) (end 77.957349 126.542135) (width 0.25) (layer "F.Cu") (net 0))
 (segment (start 77.957349 126.542135) (end 78.192561 126.583611) (width 0.25) (layer "F.Cu") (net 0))
 (segment (start 51.665524 132.930951) (end 43.848612 134.309282) (width 0.25) (layer "F.Cu") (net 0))
 (segment (start 65.460483 126.458861) (end 77.293089 126.45886) (width 0.25) (layer "F.Cu") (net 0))
 (segment (start 75.105167 115.207508) (end 75.075944 115.236733) (width 0.25) (layer "F.Cu") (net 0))
 (segment (start 43.321482 118.529207) (end 50.363032 117.287588) (width 0.25) (layer "F.Cu") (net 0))
 (segment (start 78.382207 115.413577) (end 80.275891 115.579253) (width 0.25) (layer "F.Cu") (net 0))
 (segment (start 55.849028 122.11835) (end 49.160915 123.297646) (width 0.25) (layer "F.Cu") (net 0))
 (segment (start 78.363713 115.39358) (end 75.217106 115.118283) (width 0.25) (layer "F.Cu") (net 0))
 (segment (start 64.63845 118.493075) (end 62.257202 118.493075) (width 0.25) (layer "F.Cu") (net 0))
 (segment (start 43.848612 134.309282) (end 38.466062 130.540385) (width 0.25) (layer "F.Cu") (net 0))
 (segment (start 75.740249 122.124942) (end 75.662075 122.04677) (width 0.25) (layer "F.Cu") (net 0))
 (segment (start 52.839968 119.021954) (end 53.299727 119.343882) (width 0.25) (layer "F.Cu") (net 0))
 (segment (start 22.693107 122.391573) (end 27.668522 120.58067) (width 0.25) (layer "F.Cu") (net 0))
 (segment (start 34.368315 119.060173) (end 35.48815 118.862714) (width 0.25) (layer "F.Cu") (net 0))
 (segment (start 23.358165 135.848169) (end 23.343516 135.879587) (width 0.25) (layer "F.Cu") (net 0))
 (segment (start 86.159866 116.613702) (end 80.278898 115.576728) (width 0.25) (layer "F.Cu") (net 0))
 (segment (start 61.579982 119.170293) (end 56.56972 119.17029) (width 0.25) (layer "F.Cu") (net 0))
 (segment (start 28.774207 121.096263) (end 34.368315 119.060173) (width 0.25) (layer "F.Cu") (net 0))
 (segment (start 52.839968 119.021954) (end 53.759488 119.665808) (width 0.25) (layer "F.Cu") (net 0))
 (segment (start 57.439431 123.231966) (end 55.849028 122.11835) (width 0.25) (layer "F.Cu") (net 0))
 (segment (start 85.889579 116.234112) (end 86.141368 116.593706) (width 0.25) (layer "F.Cu") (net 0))
 (segment (start 37.447968 130.719899) (end 23.358165 135.848169) (width 0.25) (layer "F.Cu") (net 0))
 (segment (start 42.128424 117.693815) (end 43.321482 118.529207) (width 0.25) (layer "F.Cu") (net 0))
 (segment (start 37.781082 120.468248) (end 40.524461 119.984515) (width 0.25) (layer "F.Cu") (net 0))
 (segment (start 62.287678 127.229111) (end 62.26317 127.253617) (width 0.25) (layer "F.Cu") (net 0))
 (segment (start 84.096804 116.249929) (end 86.154741 116.612799) (width 0.25) (layer "F.Cu") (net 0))
 (segment (start 74.168918 116.14376) (end 66.257884 116.143758) (width 0.25) (layer "F.Cu") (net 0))
 (segment (start 62.257202 118.493075) (end 61.579982 119.170293) (width 0.25) (layer "F.Cu") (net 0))
 (segment (start 56.56972 119.17029) (end 53.759488 119.665808) (width 0.25) (layer "F.Cu") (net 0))
 (segment (start 66.843501 120.698132) (end 64.63845 118.493075) (width 0.25) (layer "F.Cu") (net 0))
 (segment (start 63.844703 124.84308) (end 65.460483 126.458861) (width 0.25) (layer "F.Cu") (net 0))
 (segment (start 57.439431 123.231966) (end 57.329579 123.24158) (width 0.25) (layer "F.Cu") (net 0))
 (segment (start 64.088168 115.219247) (end 65.333373 115.219251) (width 0.25) (layer "F.Cu") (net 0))
 (segment (start 44.05046 121.309368) (end 42.509255 123.510432) (width 0.25) (layer "F.Cu") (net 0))
 (segment (start 74.530437 120.698132) (end 66.843501 120.698132) (width 0.25) (layer "F.Cu") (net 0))
 (segment (start 76.520472 127.22911) (end 62.287678 127.229111) (width 0.25) (layer "F.Cu") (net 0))
 (via (at 76.534015 127.215565) (size 0.8) (drill 0.4) (layers "F.Cu" "B.Cu") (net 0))
 (via (at 53.759488 119.665808) (size 0.8) (drill 0.4) (layers "F.Cu" "B.Cu") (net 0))
 (via (at 77.185212 122.124942) (size 0.8) (drill 0.4) (layers "F.Cu" "B.Cu") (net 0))
 (via (at 57.439431 123.231966) (size 0.8) (drill 0.4) (layers "F.Cu" "B.Cu") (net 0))
 (via (at 78.363713 115.39358) (size 0.8) (drill 0.4) (layers "F.Cu" "B.Cu") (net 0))
 (segment (start 81.368299 121.635848) (end 79.842274 119.456465) (width 0.25) (layer "B.Cu") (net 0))
 (segment (start 84.509835 122.189786) (end 83.632912 127.163066) (width 0.25) (layer "B.Cu") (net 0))
 (segment (start 70.438162 129.418619) (end 70.463165 129.443618) (width 0.25) (layer "B.Cu") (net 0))
 (segment (start 19.329929 130.699944) (end 22.327541 129.608898) (width 0.25) (layer "B.Cu") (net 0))
 (segment (start 78.947537 119.362842) (end 79.669572 119.426013) (width 0.25) (layer "B.Cu") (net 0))
 (segment (start 86.14137 116.593709) (end 87.569339 116.845495) (width 0.25) (layer "B.Cu") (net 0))
 (segment (start 55.140407 119.918049) (end 55.555381 119.423497) (width 0.25) (layer "B.Cu") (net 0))
 (segment (start 49.002201 120.108762) (end 51.269063 119.709056) (width 0.25) (layer "B.Cu") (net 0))
 (segment (start 70.463171 129.443619) (end 67.273169 129.443617) (width 0.25) (layer "B.Cu") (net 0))
 (segment (start 54.65125 122.074741) (end 55.816207 121.972822) (width 0.25) (layer "B.Cu") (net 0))
 (segment (start 78.363713 115.39358) (end 76.644067 116.836533) (width 0.25) (layer "B.Cu") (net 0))
 (segment (start 70.438163 115.219247) (end 68.988167 115.21925) (width 0.25) (layer "B.Cu") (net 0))
 (segment (start 56.276047 121.424805) (end 56.206328 120.627848) (width 0.25) (layer "B.Cu") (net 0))
 (segment (start 55.816207 121.972822) (end 56.276047 121.424805) (width 0.25) (layer "B.Cu") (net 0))
 (segment (start 92.394903 117.69637) (end 90.614614 127.792879) (width 0.25) (layer "B.Cu") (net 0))
 (segment (start 28.794424 136.236811) (end 30.692033 132.167375) (width 0.25) (layer "B.Cu") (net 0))
 (segment (start 78.389735 119.8309) (end 78.947537 119.362842) (width 0.25) (layer "B.Cu") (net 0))
 (segment (start 63.453164 126.063621) (end 62.263172 127.253618) (width 0.25) (layer "B.Cu") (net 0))
 (segment (start 50.302396 127.482509) (end 50.197649 126.888463) (width 0.25) (layer "B.Cu") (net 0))
 (segment (start 84.509835 122.189786) (end 81.368295 121.63585) (width 0.25) (layer "B.Cu") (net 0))
 (segment (start 28.131159 125.131425) (end 30.29417 124.34415) (width 0.25) (layer "B.Cu") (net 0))
 (segment (start 43.386178 128.483712) (end 42.420898 129.862275) (width 0.25) (layer "B.Cu") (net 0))
 (segment (start 79.316205 120.715009) (end 78.922846 125.211101) (width 0.25) (layer "B.Cu") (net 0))
 (segment (start 92.3949 117.696374) (end 90.966925 117.444586) (width 0.25) (layer "B.Cu") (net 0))
 (segment (start 48.381955 116.591152) (end 50.197649 126.888463) (width 0.25) (layer "B.Cu") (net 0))
 (segment (start 67.273169 129.443617) (end 67.26317 129.453619) (width 0.25) (layer "B.Cu") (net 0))
 (segment (start 59.463789 120.342855) (end 60.263171 121.013621) (width 0.25) (layer "B.Cu") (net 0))
 (segment (start 50.876608 130.595089) (end 47.735073 131.149026) (width 0.25) (layer "B.Cu") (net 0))
 (segment (start 59.063174 127.253619) (end 62.263172 127.253618) (width 0.25) (layer "B.Cu") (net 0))
 (segment (start 89.929204 131.680027) (end 89.949482 131.708987) (width 0.25) (layer "B.Cu") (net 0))
 (segment (start 90.474462 128.587723) (end 90.614614 127.792879) (width 0.25) (layer "B.Cu") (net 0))
 (segment (start 53.916294 121.458037) (end 54.65125 122.074741) (width 0.25) (layer "B.Cu") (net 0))
 (segment (start 78.320012 120.627855) (end 78.389735 119.8309) (width 0.25) (layer "B.Cu") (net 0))
 (segment (start 70.438165 115.219251) (end 70.438165 124.820533) (width 0.25) (layer "B.Cu") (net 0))
 (segment (start 78.922846 125.211101) (end 76.534015 127.215565) (width 0.25) (layer "B.Cu") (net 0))
 (segment (start 89.94948 131.708984) (end 86.807944 131.155046) (width 0.25) (layer "B.Cu") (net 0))
 (segment (start 53.759488 119.665808) (end 53.916294 121.458037) (width 0.25) (layer "B.Cu") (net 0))
 (segment (start 64.054536 115.219247) (end 64.088168 115.219248) (width 0.25) (layer "B.Cu") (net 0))
 (segment (start 70.438166 118.791123) (end 72.739992 118.791121) (width 0.25) (layer "B.Cu") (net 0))
 (segment (start 22.326167 123.508975) (end 20.963609 124.004906) (width 0.25) (layer "B.Cu") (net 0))
 (segment (start 57.437858 123.230646) (end 57.202519 120.540696) (width 0.25) (layer "B.Cu") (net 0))
 (segment (start 91.808019 121.242477) (end 94.074872 121.642189) (width 0.25) (layer "B.Cu") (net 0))
 (segment (start 64.088166 115.21925) (end 65.538165 115.219247) (width 0.25) (layer "B.Cu") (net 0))
 (segment (start 39.269515 130.417951) (end 42.420898 129.862275) (width 0.25) (layer "B.Cu") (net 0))
 (segment (start 42.128424 117.693815) (end 43.556396 117.442027) (width 0.25) (layer "B.Cu") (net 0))
 (segment (start 76.644067 116.836533) (end 76.327622 120.453537) (width 0.25) (layer "B.Cu") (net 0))
 (segment (start 50.847651 130.574809) (end 50.876611 130.595086) (width 0.25) (layer "B.Cu") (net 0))
 (segment (start 86.796361 131.163158) (end 90.474462 128.587723) (width 0.25) (layer "B.Cu") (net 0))
 (segment (start 70.438164 126.278626) (end 70.438165 124.820533) (width 0.25) (layer "B.Cu") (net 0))
 (segment (start 26.930657 121.833079) (end 25.568103 122.329006) (width 0.25) (layer "B.Cu") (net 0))
 (segment (start 28.800401 136.223992) (end 28.794423 136.23681) (width 0.25) (layer "B.Cu") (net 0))
 (segment (start 55.210131 120.715008) (end 55.140407 119.918049) (width 0.25) (layer "B.Cu") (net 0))
 (segment (start 47.735073 131.149026) (end 47.72696 131.160611) (width 0.25) (layer "B.Cu") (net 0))
 (segment (start 47.726959 131.160613) (end 50.302396 127.482509) (width 0.25) (layer "B.Cu") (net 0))
 (segment (start 83.632912 127.163066) (end 82.254347 128.128342) (width 0.25) (layer "B.Cu") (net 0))
 (segment (start 26.930657 121.833079) (end 30.566195 131.821637) (width 0.25) (layer "B.Cu") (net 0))
 (segment (start 79.842274 119.456465) (end 79.669572 119.426013) (width 0.25) (layer "B.Cu") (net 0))
 (segment (start 39.367722 124.064368) (end 42.509256 123.510434) (width 0.25) (layer "B.Cu") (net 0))
 (segment (start 31.798022 135.132949) (end 28.800401 136.223992) (width 0.25) (layer "B.Cu") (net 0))
 (segment (start 24.054748 134.354345) (end 23.343516 135.879587) (width 0.25) (layer "B.Cu") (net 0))
 (segment (start 57.439431 123.231966) (end 57.437858 123.230646) (width 0.25) (layer "B.Cu") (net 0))
 (segment (start 31.765976 135.118007) (end 31.798024 135.13295) (width 0.25) (layer "B.Cu") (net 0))
 (segment (start 78.922846 125.211101) (end 78.445627 125.611534) (width 0.25) (layer "B.Cu") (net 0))
 (segment (start 30.692033 132.167375) (end 30.566195 131.821637) (width 0.25) (layer "B.Cu") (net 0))
 (segment (start 58.198715 120.453537) (end 59.463789 120.342855) (width 0.25) (layer "B.Cu") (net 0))
 (segment (start 60.26207 119.011717) (end 64.054536 115.219247) (width 0.25) (layer "B.Cu") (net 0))
 (segment (start 42.509256 123.510434) (end 43.386178 128.483712) (width 0.25) (layer "B.Cu") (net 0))
 (segment (start 46.953983 116.842941) (end 48.381955 116.591151) (width 0.25) (layer "B.Cu") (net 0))
 (segment (start 67.263171 129.453617) (end 70.438164 126.278626) (width 0.25) (layer "B.Cu") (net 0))
 (segment (start 22.327541 129.608898) (end 24.054748 134.354345) (width 0.25) (layer "B.Cu") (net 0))
 (segment (start 86.807944 131.155046) (end 86.796359 131.163158) (width 0.25) (layer "B.Cu") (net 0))
 (segment (start 55.555381 119.423497) (end 60.26207 119.011717) (width 0.25) (layer "B.Cu") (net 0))
 (segment (start 63.453169 121.013619) (end 63.453164 126.063621) (width 0.25) (layer "B.Cu") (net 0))
 (segment (start 77.185212 122.124942) (end 77.323814 120.540692) (width 0.25) (layer "B.Cu") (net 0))
 (segment (start 20.3365 136.974051) (end 23.343516 135.879587) (width 0.25) (layer "B.Cu") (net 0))
 (segment (start 60.263168 121.013618) (end 63.453169 121.013619) (width 0.25) (layer "B.Cu") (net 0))
 (segment (start 82.254347 128.128342) (end 79.102959 127.572669) (width 0.25) (layer "B.Cu") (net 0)))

